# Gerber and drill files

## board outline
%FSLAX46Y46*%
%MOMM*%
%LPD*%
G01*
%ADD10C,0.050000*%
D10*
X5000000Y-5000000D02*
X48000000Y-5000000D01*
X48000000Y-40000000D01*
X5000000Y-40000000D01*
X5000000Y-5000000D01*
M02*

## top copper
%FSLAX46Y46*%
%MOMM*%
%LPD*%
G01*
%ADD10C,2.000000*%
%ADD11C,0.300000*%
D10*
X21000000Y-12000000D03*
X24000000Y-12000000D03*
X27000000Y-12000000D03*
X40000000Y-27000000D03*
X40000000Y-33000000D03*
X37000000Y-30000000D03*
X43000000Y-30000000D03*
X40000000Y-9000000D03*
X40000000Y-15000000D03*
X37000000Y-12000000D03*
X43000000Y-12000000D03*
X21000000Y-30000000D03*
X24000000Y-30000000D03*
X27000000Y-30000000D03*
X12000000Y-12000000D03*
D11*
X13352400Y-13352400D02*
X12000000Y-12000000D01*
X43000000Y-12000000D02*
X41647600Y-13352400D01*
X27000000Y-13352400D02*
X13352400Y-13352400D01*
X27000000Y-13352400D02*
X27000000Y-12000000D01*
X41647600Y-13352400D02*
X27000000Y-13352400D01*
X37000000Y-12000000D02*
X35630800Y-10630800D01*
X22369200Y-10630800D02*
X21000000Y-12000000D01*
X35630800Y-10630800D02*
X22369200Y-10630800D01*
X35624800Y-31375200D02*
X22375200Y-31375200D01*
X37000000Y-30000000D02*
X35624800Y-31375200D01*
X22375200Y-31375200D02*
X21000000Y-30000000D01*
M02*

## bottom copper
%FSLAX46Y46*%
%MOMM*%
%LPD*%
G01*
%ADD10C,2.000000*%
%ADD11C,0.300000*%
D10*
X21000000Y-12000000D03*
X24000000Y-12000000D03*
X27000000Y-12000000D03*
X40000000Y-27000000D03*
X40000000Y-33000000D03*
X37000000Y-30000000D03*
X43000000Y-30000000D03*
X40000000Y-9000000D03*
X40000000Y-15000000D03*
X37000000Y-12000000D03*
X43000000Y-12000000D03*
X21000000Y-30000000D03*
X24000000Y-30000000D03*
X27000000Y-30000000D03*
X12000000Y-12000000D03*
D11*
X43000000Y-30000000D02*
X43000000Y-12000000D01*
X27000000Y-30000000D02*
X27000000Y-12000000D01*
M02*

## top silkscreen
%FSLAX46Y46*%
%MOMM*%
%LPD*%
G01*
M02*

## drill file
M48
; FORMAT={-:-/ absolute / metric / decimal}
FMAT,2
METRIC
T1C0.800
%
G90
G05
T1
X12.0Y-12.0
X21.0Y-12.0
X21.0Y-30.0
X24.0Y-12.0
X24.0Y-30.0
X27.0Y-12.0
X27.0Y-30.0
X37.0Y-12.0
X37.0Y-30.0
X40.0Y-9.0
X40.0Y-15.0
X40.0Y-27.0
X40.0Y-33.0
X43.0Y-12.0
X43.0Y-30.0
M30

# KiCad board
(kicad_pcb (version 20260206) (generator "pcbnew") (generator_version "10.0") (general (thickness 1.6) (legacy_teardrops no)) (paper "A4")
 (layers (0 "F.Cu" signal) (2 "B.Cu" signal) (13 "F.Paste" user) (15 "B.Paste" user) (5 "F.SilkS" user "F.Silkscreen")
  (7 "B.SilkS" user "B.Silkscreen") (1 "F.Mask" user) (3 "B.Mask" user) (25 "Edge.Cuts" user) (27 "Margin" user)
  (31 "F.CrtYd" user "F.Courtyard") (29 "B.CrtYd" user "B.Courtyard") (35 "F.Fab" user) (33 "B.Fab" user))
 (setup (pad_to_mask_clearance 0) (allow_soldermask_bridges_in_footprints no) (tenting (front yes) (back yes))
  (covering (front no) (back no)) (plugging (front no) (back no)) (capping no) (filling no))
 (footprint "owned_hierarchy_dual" (layer "F.Cu") (at 24 12)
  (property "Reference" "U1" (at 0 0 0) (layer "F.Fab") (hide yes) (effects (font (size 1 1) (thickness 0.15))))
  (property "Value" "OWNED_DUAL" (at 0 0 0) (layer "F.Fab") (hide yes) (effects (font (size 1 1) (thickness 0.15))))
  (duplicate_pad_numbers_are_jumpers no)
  (pad "1" thru_hole circle (at -3 0) (size 2 2) (drill 0.8) (layers "*.Cu" "*.Mask") (remove_unused_layers no) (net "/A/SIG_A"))
  (pad "2" thru_hole circle (at 0 0) (size 2 2) (drill 0.8) (layers "*.Cu" "*.Mask") (remove_unused_layers no) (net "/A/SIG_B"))
  (pad "3" thru_hole circle (at 3 0) (size 2 2) (drill 0.8) (layers "*.Cu" "*.Mask") (remove_unused_layers no) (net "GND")))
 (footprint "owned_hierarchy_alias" (layer "F.Cu") (at 40 30)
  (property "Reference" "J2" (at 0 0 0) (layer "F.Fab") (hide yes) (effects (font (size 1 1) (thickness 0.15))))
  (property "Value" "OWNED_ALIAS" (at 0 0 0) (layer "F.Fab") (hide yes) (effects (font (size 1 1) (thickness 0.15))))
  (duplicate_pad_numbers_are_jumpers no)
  (pad "MP" thru_hole circle (at 0 -3) (size 2 2) (drill 0.8) (layers "*.Cu" "*.Mask") (remove_unused_layers no))
  (pad "MP" thru_hole circle (at 0 3) (size 2 2) (drill 0.8) (layers "*.Cu" "*.Mask") (remove_unused_layers no))
  (pad "R" thru_hole circle (at -3 0) (size 2 2) (drill 0.8) (layers "*.Cu" "*.Mask") (remove_unused_layers no) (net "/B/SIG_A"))
  (pad "T" thru_hole circle (at 3 0) (size 2 2) (drill 0.8) (layers "*.Cu" "*.Mask") (remove_unused_layers no) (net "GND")))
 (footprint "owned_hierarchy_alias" (layer "F.Cu") (at 40 12)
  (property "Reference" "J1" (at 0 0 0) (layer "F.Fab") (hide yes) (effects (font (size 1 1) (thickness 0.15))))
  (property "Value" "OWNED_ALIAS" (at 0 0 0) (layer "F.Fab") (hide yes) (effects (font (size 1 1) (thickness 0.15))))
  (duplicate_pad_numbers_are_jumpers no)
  (pad "MP" thru_hole circle (at 0 -3) (size 2 2) (drill 0.8) (layers "*.Cu" "*.Mask") (remove_unused_layers no))
  (pad "MP" thru_hole circle (at 0 3) (size 2 2) (drill 0.8) (layers "*.Cu" "*.Mask") (remove_unused_layers no))
  (pad "R" thru_hole circle (at -3 0) (size 2 2) (drill 0.8) (layers "*.Cu" "*.Mask") (remove_unused_layers no) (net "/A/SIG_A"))
  (pad "T" thru_hole circle (at 3 0) (size 2 2) (drill 0.8) (layers "*.Cu" "*.Mask") (remove_unused_layers no) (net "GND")))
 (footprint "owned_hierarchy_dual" (layer "F.Cu") (at 24 30)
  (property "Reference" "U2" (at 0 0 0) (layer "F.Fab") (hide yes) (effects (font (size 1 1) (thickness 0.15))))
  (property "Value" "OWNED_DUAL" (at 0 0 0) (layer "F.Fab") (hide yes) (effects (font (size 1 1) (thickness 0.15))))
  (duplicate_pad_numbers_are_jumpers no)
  (pad "1" thru_hole circle (at -3 0) (size 2 2) (drill 0.8) (layers "*.Cu" "*.Mask") (remove_unused_layers no) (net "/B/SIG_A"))
  (pad "2" thru_hole circle (at 0 0) (size 2 2) (drill 0.8) (layers "*.Cu" "*.Mask") (remove_unused_layers no) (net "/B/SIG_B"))
  (pad "3" thru_hole circle (at 3 0) (size 2 2) (drill 0.8) (layers "*.Cu" "*.Mask") (remove_unused_layers no) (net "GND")))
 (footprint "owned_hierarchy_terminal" (layer "F.Cu") (at 12 12)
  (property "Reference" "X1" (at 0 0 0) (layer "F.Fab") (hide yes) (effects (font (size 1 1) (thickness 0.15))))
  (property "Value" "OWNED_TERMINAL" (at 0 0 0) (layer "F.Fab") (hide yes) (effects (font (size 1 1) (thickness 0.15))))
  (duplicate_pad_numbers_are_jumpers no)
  (pad "1" thru_hole circle (at 0 0) (size 2 2) (drill 0.8) (layers "*.Cu" "*.Mask") (remove_unused_layers no) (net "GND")))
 (gr_rect (start 5 5) (end 48 40) (stroke (width 0.05) (type default)) (fill no) (layer "Edge.Cuts"))
 (segment (start 13.3524 13.3524) (end 12 12) (width 0.3) (layer "F.Cu") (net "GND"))
 (segment (start 43 12) (end 41.6476 13.3524) (width 0.3) (layer "F.Cu") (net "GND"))
 (segment (start 27 13.3524) (end 13.3524 13.3524) (width 0.3) (layer "F.Cu") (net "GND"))
 (segment (start 27 13.3524) (end 27 12) (width 0.3) (layer "F.Cu") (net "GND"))
 (segment (start 41.6476 13.3524) (end 27 13.3524) (width 0.3) (layer "F.Cu") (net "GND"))
 (segment (start 43 30) (end 43 12) (width 0.3) (layer "B.Cu") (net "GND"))
 (segment (start 27 30) (end 27 12) (width 0.3) (layer "B.Cu") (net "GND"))
 (segment (start 37 12) (end 35.6308 10.6308) (width 0.3) (layer "F.Cu") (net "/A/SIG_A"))
 (segment (start 22.3692 10.6308) (end 21 12) (width 0.3) (layer "F.Cu") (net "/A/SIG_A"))
 (segment (start 35.6308 10.6308) (end 22.3692 10.6308) (width 0.3) (layer "F.Cu") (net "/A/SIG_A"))
 (segment (start 35.6248 31.3752) (end 22.3752 31.3752) (width 0.3) (layer "F.Cu") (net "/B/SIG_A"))
 (segment (start 37 30) (end 35.6248 31.3752) (width 0.3) (layer "F.Cu") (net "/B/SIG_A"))
 (segment (start 22.3752 31.3752) (end 21 30) (width 0.3) (layer "F.Cu") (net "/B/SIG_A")))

